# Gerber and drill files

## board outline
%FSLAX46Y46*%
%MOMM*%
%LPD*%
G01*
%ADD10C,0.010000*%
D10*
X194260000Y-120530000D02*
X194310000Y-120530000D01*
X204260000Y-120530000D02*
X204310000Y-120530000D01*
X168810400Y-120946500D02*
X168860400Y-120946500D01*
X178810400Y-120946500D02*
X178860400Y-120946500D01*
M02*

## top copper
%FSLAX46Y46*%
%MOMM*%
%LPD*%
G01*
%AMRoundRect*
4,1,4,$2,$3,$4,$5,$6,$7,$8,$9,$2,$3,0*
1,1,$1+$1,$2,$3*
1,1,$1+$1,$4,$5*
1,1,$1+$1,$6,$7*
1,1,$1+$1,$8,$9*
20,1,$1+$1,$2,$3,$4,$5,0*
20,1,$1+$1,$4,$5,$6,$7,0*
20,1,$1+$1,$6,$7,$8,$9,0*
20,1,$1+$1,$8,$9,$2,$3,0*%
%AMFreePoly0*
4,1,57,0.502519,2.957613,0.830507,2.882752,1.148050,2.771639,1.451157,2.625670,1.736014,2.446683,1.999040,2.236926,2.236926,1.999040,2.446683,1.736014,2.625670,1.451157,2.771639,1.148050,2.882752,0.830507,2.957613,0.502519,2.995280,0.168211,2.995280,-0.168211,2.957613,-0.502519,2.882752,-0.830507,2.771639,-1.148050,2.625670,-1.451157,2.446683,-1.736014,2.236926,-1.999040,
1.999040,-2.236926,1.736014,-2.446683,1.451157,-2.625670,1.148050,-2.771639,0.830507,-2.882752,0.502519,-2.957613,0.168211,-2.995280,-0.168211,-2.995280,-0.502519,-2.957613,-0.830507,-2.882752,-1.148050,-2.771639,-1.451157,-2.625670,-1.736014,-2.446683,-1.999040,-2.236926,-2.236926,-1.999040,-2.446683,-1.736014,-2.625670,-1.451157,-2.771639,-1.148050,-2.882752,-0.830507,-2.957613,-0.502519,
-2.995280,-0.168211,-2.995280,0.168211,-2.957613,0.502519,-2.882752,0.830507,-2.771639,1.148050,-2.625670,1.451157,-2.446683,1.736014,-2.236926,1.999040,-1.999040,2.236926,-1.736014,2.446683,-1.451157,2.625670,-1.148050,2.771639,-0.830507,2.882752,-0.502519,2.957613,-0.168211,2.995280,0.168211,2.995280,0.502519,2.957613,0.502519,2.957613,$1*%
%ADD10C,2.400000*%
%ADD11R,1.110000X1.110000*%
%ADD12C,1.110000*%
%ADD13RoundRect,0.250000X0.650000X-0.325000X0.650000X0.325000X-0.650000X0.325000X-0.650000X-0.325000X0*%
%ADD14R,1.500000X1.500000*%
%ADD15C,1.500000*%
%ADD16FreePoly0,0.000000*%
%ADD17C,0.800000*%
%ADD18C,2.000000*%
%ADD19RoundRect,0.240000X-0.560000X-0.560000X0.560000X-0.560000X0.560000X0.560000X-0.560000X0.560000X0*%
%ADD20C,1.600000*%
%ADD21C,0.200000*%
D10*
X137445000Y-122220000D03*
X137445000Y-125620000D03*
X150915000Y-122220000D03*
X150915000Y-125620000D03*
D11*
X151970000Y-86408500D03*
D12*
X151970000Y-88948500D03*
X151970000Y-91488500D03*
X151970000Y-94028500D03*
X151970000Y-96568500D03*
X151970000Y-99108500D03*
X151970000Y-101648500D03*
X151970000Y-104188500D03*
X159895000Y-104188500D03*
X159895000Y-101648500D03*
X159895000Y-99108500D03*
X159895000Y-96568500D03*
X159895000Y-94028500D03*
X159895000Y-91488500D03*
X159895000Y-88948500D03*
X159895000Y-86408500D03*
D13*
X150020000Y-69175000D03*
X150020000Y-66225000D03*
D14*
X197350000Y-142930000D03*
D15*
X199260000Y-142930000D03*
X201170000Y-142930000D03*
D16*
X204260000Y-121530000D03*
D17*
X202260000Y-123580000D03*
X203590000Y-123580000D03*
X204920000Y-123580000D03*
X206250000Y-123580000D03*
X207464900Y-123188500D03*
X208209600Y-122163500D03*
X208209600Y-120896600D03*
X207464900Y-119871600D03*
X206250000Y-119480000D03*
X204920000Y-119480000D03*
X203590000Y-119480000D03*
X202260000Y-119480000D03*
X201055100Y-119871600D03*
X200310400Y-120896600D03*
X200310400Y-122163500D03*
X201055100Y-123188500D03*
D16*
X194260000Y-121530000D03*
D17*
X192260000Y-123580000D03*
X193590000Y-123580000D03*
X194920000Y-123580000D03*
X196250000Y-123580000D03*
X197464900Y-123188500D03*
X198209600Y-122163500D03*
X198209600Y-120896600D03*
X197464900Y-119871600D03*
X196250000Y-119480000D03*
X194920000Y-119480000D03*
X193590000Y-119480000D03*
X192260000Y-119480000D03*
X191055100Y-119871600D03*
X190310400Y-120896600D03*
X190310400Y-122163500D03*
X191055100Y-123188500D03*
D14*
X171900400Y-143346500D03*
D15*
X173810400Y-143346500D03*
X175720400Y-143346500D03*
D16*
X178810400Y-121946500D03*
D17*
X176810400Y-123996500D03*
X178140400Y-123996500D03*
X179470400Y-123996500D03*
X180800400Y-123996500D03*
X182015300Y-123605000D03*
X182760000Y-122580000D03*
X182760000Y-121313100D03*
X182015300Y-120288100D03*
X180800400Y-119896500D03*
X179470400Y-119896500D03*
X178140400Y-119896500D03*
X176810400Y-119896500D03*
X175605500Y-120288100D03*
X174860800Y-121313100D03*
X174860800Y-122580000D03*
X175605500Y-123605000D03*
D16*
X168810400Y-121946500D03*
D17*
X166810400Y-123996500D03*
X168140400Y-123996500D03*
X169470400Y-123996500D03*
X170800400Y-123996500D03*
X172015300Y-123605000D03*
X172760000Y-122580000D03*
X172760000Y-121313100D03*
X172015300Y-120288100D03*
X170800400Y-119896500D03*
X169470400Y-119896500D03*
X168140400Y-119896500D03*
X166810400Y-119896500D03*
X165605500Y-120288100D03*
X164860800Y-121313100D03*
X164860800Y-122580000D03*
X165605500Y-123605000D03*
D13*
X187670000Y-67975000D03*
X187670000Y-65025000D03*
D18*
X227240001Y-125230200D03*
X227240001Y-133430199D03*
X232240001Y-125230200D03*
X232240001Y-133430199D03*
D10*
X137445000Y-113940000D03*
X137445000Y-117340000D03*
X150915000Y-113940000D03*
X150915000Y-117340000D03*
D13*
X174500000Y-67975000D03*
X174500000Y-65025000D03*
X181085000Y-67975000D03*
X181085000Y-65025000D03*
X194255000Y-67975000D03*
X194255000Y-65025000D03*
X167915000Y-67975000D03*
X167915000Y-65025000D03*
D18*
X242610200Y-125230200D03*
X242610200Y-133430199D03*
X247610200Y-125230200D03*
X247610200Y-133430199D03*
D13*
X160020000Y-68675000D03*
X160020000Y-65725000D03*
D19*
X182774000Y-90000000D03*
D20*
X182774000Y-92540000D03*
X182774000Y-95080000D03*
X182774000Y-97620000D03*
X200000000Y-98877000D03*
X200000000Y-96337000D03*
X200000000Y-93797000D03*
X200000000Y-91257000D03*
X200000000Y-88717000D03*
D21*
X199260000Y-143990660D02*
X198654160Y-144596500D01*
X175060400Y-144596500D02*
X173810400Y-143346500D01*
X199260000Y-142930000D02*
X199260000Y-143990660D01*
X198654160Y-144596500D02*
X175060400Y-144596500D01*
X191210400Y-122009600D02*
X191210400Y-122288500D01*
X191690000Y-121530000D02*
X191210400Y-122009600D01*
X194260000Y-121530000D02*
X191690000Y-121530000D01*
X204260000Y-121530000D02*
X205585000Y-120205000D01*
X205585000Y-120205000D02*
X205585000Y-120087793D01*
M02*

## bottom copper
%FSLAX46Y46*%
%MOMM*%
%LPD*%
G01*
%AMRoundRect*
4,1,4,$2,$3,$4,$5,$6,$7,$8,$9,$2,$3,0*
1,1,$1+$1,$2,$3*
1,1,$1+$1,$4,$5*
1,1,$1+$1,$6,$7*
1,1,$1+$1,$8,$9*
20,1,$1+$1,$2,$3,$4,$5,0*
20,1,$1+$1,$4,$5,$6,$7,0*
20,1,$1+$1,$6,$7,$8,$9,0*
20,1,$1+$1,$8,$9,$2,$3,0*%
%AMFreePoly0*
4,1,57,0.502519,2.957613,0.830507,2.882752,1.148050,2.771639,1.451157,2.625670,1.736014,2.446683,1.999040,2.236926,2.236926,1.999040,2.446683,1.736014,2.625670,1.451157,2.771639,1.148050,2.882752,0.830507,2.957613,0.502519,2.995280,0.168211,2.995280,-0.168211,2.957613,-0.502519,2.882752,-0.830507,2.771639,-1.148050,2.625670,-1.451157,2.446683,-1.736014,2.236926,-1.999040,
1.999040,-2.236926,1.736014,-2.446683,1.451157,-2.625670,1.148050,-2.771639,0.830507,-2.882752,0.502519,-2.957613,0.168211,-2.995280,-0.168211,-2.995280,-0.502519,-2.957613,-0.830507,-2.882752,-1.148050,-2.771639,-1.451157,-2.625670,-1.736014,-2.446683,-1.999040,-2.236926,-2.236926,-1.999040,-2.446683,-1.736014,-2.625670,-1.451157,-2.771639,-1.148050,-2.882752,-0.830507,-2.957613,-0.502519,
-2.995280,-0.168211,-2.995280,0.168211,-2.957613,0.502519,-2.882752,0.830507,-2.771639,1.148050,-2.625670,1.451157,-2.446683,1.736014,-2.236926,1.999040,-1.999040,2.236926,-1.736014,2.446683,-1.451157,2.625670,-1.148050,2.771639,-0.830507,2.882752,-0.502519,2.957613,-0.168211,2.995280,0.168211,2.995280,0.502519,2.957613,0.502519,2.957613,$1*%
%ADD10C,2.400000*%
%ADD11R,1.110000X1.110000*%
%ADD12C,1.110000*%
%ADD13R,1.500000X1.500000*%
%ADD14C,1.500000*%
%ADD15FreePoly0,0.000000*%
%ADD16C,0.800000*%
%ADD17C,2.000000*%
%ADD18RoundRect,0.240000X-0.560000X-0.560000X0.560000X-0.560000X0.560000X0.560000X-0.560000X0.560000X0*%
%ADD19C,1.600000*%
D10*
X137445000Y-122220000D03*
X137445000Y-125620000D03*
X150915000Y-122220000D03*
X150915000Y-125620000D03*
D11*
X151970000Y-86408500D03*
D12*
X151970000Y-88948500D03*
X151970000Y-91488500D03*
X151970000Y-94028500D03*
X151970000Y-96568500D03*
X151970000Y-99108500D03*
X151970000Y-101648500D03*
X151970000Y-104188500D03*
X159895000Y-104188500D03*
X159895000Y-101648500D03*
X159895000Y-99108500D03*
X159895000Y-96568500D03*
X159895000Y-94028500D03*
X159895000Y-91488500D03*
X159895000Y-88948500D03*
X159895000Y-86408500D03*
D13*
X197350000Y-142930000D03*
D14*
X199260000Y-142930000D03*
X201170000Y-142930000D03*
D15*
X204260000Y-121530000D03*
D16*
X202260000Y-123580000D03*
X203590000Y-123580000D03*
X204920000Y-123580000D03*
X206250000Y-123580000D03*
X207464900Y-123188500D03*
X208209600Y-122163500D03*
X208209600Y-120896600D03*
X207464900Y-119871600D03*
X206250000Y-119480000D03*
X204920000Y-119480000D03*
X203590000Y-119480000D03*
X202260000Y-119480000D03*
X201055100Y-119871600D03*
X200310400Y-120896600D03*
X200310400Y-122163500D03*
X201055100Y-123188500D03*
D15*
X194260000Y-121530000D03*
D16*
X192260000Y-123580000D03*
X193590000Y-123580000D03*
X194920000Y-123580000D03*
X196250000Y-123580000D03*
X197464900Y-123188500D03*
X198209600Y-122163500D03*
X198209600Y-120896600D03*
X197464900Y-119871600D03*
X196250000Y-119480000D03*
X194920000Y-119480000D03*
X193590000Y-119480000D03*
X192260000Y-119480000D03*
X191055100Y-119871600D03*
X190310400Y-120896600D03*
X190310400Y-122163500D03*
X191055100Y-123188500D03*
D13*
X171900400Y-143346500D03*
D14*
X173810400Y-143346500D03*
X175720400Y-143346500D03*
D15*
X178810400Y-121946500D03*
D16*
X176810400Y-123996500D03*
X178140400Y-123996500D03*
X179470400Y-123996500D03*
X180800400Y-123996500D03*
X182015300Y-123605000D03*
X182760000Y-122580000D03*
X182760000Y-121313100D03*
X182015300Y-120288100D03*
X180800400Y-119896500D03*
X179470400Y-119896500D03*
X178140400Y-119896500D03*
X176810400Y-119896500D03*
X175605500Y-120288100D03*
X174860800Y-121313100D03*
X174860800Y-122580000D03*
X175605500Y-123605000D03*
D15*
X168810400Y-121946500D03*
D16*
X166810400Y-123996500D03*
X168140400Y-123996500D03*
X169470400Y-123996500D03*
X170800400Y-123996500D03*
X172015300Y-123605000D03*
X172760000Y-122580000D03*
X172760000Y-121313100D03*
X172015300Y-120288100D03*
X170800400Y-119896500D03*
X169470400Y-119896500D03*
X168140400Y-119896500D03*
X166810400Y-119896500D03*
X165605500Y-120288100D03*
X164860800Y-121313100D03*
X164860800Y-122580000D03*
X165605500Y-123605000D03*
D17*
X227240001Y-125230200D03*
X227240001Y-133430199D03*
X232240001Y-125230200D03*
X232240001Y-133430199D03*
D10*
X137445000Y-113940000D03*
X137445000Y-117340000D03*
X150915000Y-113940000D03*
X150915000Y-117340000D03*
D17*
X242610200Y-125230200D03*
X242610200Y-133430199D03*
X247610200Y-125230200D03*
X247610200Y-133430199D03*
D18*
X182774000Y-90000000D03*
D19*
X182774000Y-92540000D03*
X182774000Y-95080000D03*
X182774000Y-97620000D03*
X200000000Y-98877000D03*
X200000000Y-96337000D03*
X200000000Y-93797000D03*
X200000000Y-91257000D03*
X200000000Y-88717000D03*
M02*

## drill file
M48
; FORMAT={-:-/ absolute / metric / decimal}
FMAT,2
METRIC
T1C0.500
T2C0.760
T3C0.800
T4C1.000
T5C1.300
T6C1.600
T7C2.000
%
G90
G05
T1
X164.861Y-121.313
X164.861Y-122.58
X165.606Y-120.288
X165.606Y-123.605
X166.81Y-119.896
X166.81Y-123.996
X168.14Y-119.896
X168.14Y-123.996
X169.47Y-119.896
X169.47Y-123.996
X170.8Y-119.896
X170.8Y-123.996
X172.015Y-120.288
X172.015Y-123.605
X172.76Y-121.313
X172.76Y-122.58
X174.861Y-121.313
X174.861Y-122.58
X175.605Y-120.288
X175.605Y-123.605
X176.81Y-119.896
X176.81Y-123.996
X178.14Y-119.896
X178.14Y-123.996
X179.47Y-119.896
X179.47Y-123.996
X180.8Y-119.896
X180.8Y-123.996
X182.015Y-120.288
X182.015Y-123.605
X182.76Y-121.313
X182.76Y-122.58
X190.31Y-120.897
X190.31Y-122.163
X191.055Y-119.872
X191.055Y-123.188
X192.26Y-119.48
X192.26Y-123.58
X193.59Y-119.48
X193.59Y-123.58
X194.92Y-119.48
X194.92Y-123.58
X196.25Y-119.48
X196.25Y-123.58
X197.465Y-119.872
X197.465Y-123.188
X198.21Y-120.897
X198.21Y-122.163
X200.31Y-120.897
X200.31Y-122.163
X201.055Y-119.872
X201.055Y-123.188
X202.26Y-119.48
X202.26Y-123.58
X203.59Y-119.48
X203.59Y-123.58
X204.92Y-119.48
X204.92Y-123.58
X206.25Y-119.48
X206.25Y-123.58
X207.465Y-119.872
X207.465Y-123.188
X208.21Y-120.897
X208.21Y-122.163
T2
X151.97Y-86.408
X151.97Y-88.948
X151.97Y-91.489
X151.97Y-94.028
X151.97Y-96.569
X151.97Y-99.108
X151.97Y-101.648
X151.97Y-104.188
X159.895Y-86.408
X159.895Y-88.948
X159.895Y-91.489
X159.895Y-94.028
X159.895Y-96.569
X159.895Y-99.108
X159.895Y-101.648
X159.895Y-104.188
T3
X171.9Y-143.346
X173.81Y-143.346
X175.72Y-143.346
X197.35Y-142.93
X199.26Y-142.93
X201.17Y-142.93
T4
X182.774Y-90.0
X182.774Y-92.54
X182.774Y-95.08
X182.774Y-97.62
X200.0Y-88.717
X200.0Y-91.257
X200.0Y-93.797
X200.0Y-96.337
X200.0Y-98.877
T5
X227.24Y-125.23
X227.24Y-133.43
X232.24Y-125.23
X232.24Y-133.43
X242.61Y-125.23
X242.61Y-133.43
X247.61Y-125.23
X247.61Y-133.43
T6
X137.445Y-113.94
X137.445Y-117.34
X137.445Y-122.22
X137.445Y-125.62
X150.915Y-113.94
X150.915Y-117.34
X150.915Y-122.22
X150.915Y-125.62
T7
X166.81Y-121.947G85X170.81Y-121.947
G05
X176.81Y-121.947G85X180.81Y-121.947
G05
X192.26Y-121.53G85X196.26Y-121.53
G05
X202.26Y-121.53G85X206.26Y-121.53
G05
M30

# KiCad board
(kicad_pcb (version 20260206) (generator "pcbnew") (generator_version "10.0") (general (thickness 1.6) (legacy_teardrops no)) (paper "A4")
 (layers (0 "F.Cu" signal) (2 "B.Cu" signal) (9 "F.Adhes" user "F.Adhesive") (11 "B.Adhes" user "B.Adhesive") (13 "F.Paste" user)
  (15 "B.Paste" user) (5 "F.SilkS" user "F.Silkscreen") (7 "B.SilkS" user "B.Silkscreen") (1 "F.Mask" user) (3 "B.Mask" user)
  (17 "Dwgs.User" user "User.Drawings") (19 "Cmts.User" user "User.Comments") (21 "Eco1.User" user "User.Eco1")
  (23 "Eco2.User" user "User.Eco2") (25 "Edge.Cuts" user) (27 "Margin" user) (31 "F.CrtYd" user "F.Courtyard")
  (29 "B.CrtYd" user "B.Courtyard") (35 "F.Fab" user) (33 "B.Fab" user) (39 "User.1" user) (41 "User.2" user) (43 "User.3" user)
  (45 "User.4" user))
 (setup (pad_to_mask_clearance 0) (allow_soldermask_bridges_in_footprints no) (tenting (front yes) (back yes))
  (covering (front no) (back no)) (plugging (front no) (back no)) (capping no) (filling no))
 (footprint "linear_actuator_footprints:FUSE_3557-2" (layer "F.Cu") (at 144.18 123.92)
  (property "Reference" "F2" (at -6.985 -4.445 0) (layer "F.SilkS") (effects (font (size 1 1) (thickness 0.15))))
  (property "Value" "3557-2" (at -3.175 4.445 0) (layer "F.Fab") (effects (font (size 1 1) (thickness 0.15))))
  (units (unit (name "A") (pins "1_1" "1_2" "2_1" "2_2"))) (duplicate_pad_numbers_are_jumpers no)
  (pad "1_1" thru_hole circle (at -6.735 -1.7) (size 2.4 2.4) (drill 1.6) (layers "*.Cu" "*.Mask") (remove_unused_layers no)
   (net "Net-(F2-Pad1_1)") (solder_mask_margin 0.102))
  (pad "1_2" thru_hole circle (at -6.735 1.7) (size 2.4 2.4) (drill 1.6) (layers "*.Cu" "*.Mask") (remove_unused_layers no)
   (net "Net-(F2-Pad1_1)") (solder_mask_margin 0.102))
  (pad "2_1" thru_hole circle (at 6.735 -1.7) (size 2.4 2.4) (drill 1.6) (layers "*.Cu" "*.Mask") (remove_unused_layers no)
   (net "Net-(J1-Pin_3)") (solder_mask_margin 0.102))
  (pad "2_2" thru_hole circle (at 6.735 1.7) (size 2.4 2.4) (drill 1.6) (layers "*.Cu" "*.Mask") (remove_unused_layers no)
   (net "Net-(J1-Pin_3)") (solder_mask_margin 0.102)))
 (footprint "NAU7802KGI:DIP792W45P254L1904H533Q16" (layer "F.Cu") (at 155.9325 95.2985)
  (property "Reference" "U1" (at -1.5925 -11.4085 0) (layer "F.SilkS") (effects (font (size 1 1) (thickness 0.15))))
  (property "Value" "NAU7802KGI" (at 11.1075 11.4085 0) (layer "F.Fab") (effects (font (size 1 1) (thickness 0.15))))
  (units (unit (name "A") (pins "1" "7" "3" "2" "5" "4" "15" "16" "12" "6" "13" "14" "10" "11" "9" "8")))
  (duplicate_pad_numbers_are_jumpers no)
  (pad "1" thru_hole rect (at -3.9625 -8.89) (size 1.11 1.11) (drill 0.76) (layers "*.Cu" "*.Mask") (remove_unused_layers no) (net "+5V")
   (solder_mask_margin 0.102))
  (pad "2" thru_hole circle (at -3.9625 -6.35) (size 1.11 1.11) (drill 0.76) (layers "*.Cu" "*.Mask") (remove_unused_layers no) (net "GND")
   (solder_mask_margin 0.102))
  (pad "3" thru_hole circle (at -3.9625 -3.81) (size 1.11 1.11) (drill 0.76) (layers "*.Cu" "*.Mask") (remove_unused_layers no)
   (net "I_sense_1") (solder_mask_margin 0.102))
  (pad "4" thru_hole circle (at -3.9625 -1.27) (size 1.11 1.11) (drill 0.76) (layers "*.Cu" "*.Mask") (remove_unused_layers no) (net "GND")
   (solder_mask_margin 0.102))
  (pad "5" thru_hole circle (at -3.9625 1.27) (size 1.11 1.11) (drill 0.76) (layers "*.Cu" "*.Mask") (remove_unused_layers no)
   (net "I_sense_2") (solder_mask_margin 0.102))
  (pad "6" thru_hole circle (at -3.9625 3.81) (size 1.11 1.11) (drill 0.76) (layers "*.Cu" "*.Mask") (remove_unused_layers no)
   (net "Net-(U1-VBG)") (solder_mask_margin 0.102))
  (pad "7" thru_hole circle (at -3.9625 6.35) (size 1.11 1.11) (drill 0.76) (layers "*.Cu" "*.Mask") (remove_unused_layers no) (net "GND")
   (solder_mask_margin 0.102))
  (pad "8" thru_hole circle (at -3.9625 8.89) (size 1.11 1.11) (drill 0.76) (layers "*.Cu" "*.Mask") (remove_unused_layers no) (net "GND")
   (solder_mask_margin 0.102))
  (pad "9" thru_hole circle (at 3.9625 8.89) (size 1.11 1.11) (drill 0.76) (layers "*.Cu" "*.Mask") (remove_unused_layers no) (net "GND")
   (solder_mask_margin 0.102))
  (pad "10" thru_hole circle (at 3.9625 6.35) (size 1.11 1.11) (drill 0.76) (layers "*.Cu" "*.Mask") (remove_unused_layers no)
   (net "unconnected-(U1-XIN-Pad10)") (solder_mask_margin 0.102))
  (pad "11" thru_hole circle (at 3.9625 3.81) (size 1.11 1.11) (drill 0.76) (layers "*.Cu" "*.Mask") (remove_unused_layers no)
   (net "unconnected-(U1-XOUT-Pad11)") (solder_mask_margin 0.102))
  (pad "12" thru_hole circle (at 3.9625 1.27) (size 1.11 1.11) (drill 0.76) (layers "*.Cu" "*.Mask") (remove_unused_layers no)
   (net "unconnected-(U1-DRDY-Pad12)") (solder_mask_margin 0.102))
  (pad "13" thru_hole circle (at 3.9625 -1.27) (size 1.11 1.11) (drill 0.76) (layers "*.Cu" "*.Mask") (remove_unused_layers no)
   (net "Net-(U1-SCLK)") (solder_mask_margin 0.102))
  (pad "14" thru_hole circle (at 3.9625 -3.81) (size 1.11 1.11) (drill 0.76) (layers "*.Cu" "*.Mask") (remove_unused_layers no)
   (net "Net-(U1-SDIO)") (solder_mask_margin 0.102))
  (pad "15" thru_hole circle (at 3.9625 -6.35) (size 1.11 1.11) (drill 0.76) (layers "*.Cu" "*.Mask") (remove_unused_layers no) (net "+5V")
   (solder_mask_margin 0.102))
  (pad "16" thru_hole circle (at 3.9625 -8.89) (size 1.11 1.11) (drill 0.76) (layers "*.Cu" "*.Mask") (remove_unused_layers no)
   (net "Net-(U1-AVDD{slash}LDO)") (solder_mask_margin 0.102)))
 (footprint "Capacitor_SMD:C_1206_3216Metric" (layer "F.Cu") (at 150.02 67.7 90)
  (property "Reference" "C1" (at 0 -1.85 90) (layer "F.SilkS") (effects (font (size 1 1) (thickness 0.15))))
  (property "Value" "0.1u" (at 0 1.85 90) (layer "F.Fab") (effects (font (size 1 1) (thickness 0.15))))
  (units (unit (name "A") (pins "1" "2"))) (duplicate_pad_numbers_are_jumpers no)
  (pad "1" smd roundrect (at -1.475 0 90) (size 1.15 1.8) (layers "F.Cu" "F.Mask" "F.Paste") (roundrect_rratio 0.217391) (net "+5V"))
  (pad "2" smd roundrect (at 1.475 0 90) (size 1.15 1.8) (layers "F.Cu" "F.Mask" "F.Paste") (roundrect_rratio 0.217391) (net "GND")))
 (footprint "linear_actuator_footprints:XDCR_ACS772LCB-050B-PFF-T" (layer "F.Cu") (at 199.26 132.23)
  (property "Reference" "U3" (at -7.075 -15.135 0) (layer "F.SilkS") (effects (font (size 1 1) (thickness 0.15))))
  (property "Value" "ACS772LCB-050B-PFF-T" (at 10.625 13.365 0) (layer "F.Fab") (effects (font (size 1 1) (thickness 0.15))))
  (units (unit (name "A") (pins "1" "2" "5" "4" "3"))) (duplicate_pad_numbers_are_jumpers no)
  (fp_line (start -5 -11.7) (end -4.95 -11.7) (stroke (width 0.01) (type solid)) (layer "Edge.Cuts"))
  (fp_line (start 5 -11.7) (end 5.05 -11.7) (stroke (width 0.01) (type solid)) (layer "Edge.Cuts"))
  (pad "1" thru_hole rect (at -1.91 10.7) (size 1.5 1.5) (drill 0.8) (layers "*.Cu" "*.Mask") (remove_unused_layers no) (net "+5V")
   (solder_mask_margin 0.102))
  (pad "2" thru_hole circle (at 0 10.7) (size 1.5 1.5) (drill 0.8) (layers "*.Cu" "*.Mask") (remove_unused_layers no) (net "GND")
   (solder_mask_margin 0.102))
  (pad "3" thru_hole circle (at 1.91 10.7) (size 1.5 1.5) (drill 0.8) (layers "*.Cu" "*.Mask") (remove_unused_layers no) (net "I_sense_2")
   (solder_mask_margin 0.102))
  (pad "4" thru_hole custom (at 5 -10.7) (size 6 3) (drill oval 6 2) (layers "*.Cu") (remove_unused_layers no) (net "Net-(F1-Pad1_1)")
   (thermal_bridge_angle 90) (options (clearance outline) (anchor circle)) (primitives))
  (pad "4_1" thru_hole circle (at 3 -8.65) (size 0.8 0.8) (drill 0.5) (layers "*.Cu" "*.Mask") (remove_unused_layers no)
   (solder_mask_margin 0.102))
  (pad "4_2" thru_hole circle (at 4.33 -8.65) (size 0.8 0.8) (drill 0.5) (layers "*.Cu" "*.Mask") (remove_unused_layers no)
   (solder_mask_margin 0.102))
  (pad "4_3" thru_hole circle (at 5.66 -8.65) (size 0.8 0.8) (drill 0.5) (layers "*.Cu" "*.Mask") (remove_unused_layers no)
   (solder_mask_margin 0.102))
  (pad "4_4" thru_hole circle (at 6.99 -8.65) (size 0.8 0.8) (drill 0.5) (layers "*.Cu" "*.Mask") (remove_unused_layers no)
   (solder_mask_margin 0.102))
  (pad "4_5" thru_hole circle (at 8.2049 -9.0415) (size 0.8 0.8) (drill 0.5) (layers "*.Cu" "*.Mask") (remove_unused_layers no)
   (solder_mask_margin 0.102))
  (pad "4_6" thru_hole circle (at 8.9496 -10.0665) (size 0.8 0.8) (drill 0.5) (layers "*.Cu" "*.Mask") (remove_unused_layers no)
   (solder_mask_margin 0.102))
  (pad "4_7" thru_hole circle (at 8.9496 -11.3334) (size 0.8 0.8) (drill 0.5) (layers "*.Cu" "*.Mask") (remove_unused_layers no)
   (solder_mask_margin 0.102))
  (pad "4_8" thru_hole circle (at 8.2049 -12.3584) (size 0.8 0.8) (drill 0.5) (layers "*.Cu" "*.Mask") (remove_unused_layers no)
   (solder_mask_margin 0.102))
  (pad "4_9" thru_hole circle (at 6.99 -12.75) (size 0.8 0.8) (drill 0.5) (layers "*.Cu" "*.Mask") (remove_unused_layers no)
   (solder_mask_margin 0.102))
  (pad "4_10" thru_hole circle (at 5.66 -12.75) (size 0.8 0.8) (drill 0.5) (layers "*.Cu" "*.Mask") (remove_unused_layers no)
   (solder_mask_margin 0.102))
  (pad "4_11" thru_hole circle (at 4.33 -12.75) (size 0.8 0.8) (drill 0.5) (layers "*.Cu" "*.Mask") (remove_unused_layers no)
   (solder_mask_margin 0.102))
  (pad "4_12" thru_hole circle (at 3 -12.75) (size 0.8 0.8) (drill 0.5) (layers "*.Cu" "*.Mask") (remove_unused_layers no)
   (solder_mask_margin 0.102))
  (pad "4_13" thru_hole circle (at 1.7951 -12.3584) (size 0.8 0.8) (drill 0.5) (layers "*.Cu" "*.Mask") (remove_unused_layers no)
   (solder_mask_margin 0.102))
  (pad "4_14" thru_hole circle (at 1.0504 -11.3334) (size 0.8 0.8) (drill 0.5) (layers "*.Cu" "*.Mask") (remove_unused_layers no)
   (solder_mask_margin 0.102))
  (pad "4_15" thru_hole circle (at 1.0504 -10.0665) (size 0.8 0.8) (drill 0.5) (layers "*.Cu" "*.Mask") (remove_unused_layers no)
   (solder_mask_margin 0.102))
  (pad "4_16" thru_hole circle (at 1.7951 -9.0415) (size 0.8 0.8) (drill 0.5) (layers "*.Cu" "*.Mask") (remove_unused_layers no)
   (solder_mask_margin 0.102))
  (pad "5" thru_hole custom (at -5 -10.7) (size 6 3) (drill oval 6 2) (layers "*.Cu") (remove_unused_layers no) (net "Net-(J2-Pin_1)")
   (thermal_bridge_angle 90) (options (clearance outline) (anchor circle)) (primitives))
  (pad "5_1" thru_hole circle (at -7 -8.65) (size 0.8 0.8) (drill 0.5) (layers "*.Cu" "*.Mask") (remove_unused_layers no)
   (solder_mask_margin 0.102))
  (pad "5_2" thru_hole circle (at -5.67 -8.65) (size 0.8 0.8) (drill 0.5) (layers "*.Cu" "*.Mask") (remove_unused_layers no)
   (solder_mask_margin 0.102))
  (pad "5_3" thru_hole circle (at -4.34 -8.65) (size 0.8 0.8) (drill 0.5) (layers "*.Cu" "*.Mask") (remove_unused_layers no)
   (solder_mask_margin 0.102))
  (pad "5_4" thru_hole circle (at -3.01 -8.65) (size 0.8 0.8) (drill 0.5) (layers "*.Cu" "*.Mask") (remove_unused_layers no)
   (solder_mask_margin 0.102))
  (pad "5_5" thru_hole circle (at -1.7951 -9.0415) (size 0.8 0.8) (drill 0.5) (layers "*.Cu" "*.Mask") (remove_unused_layers no)
   (solder_mask_margin 0.102))
  (pad "5_6" thru_hole circle (at -1.0504 -10.0665) (size 0.8 0.8) (drill 0.5) (layers "*.Cu" "*.Mask") (remove_unused_layers no)
   (solder_mask_margin 0.102))
  (pad "5_7" thru_hole circle (at -1.0504 -11.3334) (size 0.8 0.8) (drill 0.5) (layers "*.Cu" "*.Mask") (remove_unused_layers no)
   (solder_mask_margin 0.102))
  (pad "5_8" thru_hole circle (at -1.7951 -12.3584) (size 0.8 0.8) (drill 0.5) (layers "*.Cu" "*.Mask") (remove_unused_layers no)
   (solder_mask_margin 0.102))
  (pad "5_9" thru_hole circle (at -3.01 -12.75) (size 0.8 0.8) (drill 0.5) (layers "*.Cu" "*.Mask") (remove_unused_layers no)
   (solder_mask_margin 0.102))
  (pad "5_10" thru_hole circle (at -4.34 -12.75) (size 0.8 0.8) (drill 0.5) (layers "*.Cu" "*.Mask") (remove_unused_layers no)
   (solder_mask_margin 0.102))
  (pad "5_11" thru_hole circle (at -5.67 -12.75) (size 0.8 0.8) (drill 0.5) (layers "*.Cu" "*.Mask") (remove_unused_layers no)
   (solder_mask_margin 0.102))
  (pad "5_12" thru_hole circle (at -7 -12.75) (size 0.8 0.8) (drill 0.5) (layers "*.Cu" "*.Mask") (remove_unused_layers no)
   (solder_mask_margin 0.102))
  (pad "5_13" thru_hole circle (at -8.2049 -12.3584) (size 0.8 0.8) (drill 0.5) (layers "*.Cu" "*.Mask") (remove_unused_layers no)
   (solder_mask_margin 0.102))
  (pad "5_14" thru_hole circle (at -8.9496 -11.3334) (size 0.8 0.8) (drill 0.5) (layers "*.Cu" "*.Mask") (remove_unused_layers no)
   (solder_mask_margin 0.102))
  (pad "5_15" thru_hole circle (at -8.9496 -10.0665) (size 0.8 0.8) (drill 0.5) (layers "*.Cu" "*.Mask") (remove_unused_layers no)
   (solder_mask_margin 0.102))
  (pad "5_16" thru_hole circle (at -8.2049 -9.0415) (size 0.8 0.8) (drill 0.5) (layers "*.Cu" "*.Mask") (remove_unused_layers no)
   (solder_mask_margin 0.102)))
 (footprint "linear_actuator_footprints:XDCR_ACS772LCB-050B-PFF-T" (layer "F.Cu") (at 173.8104 132.6465)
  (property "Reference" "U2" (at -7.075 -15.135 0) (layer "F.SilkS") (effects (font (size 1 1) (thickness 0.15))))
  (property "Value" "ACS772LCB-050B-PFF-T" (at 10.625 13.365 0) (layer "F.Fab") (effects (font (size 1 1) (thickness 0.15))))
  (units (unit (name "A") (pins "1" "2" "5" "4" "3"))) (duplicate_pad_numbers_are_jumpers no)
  (fp_line (start -5 -11.7) (end -4.95 -11.7) (stroke (width 0.01) (type solid)) (layer "Edge.Cuts"))
  (fp_line (start 5 -11.7) (end 5.05 -11.7) (stroke (width 0.01) (type solid)) (layer "Edge.Cuts"))
  (pad "1" thru_hole rect (at -1.91 10.7) (size 1.5 1.5) (drill 0.8) (layers "*.Cu" "*.Mask") (remove_unused_layers no) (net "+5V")
   (solder_mask_margin 0.102))
  (pad "2" thru_hole circle (at 0 10.7) (size 1.5 1.5) (drill 0.8) (layers "*.Cu" "*.Mask") (remove_unused_layers no) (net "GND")
   (solder_mask_margin 0.102))
  (pad "3" thru_hole circle (at 1.91 10.7) (size 1.5 1.5) (drill 0.8) (layers "*.Cu" "*.Mask") (remove_unused_layers no) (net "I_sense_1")
   (solder_mask_margin 0.102))
  (pad "4" thru_hole custom (at 5 -10.7) (size 6 3) (drill oval 6 2) (layers "*.Cu") (remove_unused_layers no) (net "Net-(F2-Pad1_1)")
   (thermal_bridge_angle 90) (options (clearance outline) (anchor circle)) (primitives))
  (pad "4_1" thru_hole circle (at 3 -8.65) (size 0.8 0.8) (drill 0.5) (layers "*.Cu" "*.Mask") (remove_unused_layers no)
   (solder_mask_margin 0.102))
  (pad "4_2" thru_hole circle (at 4.33 -8.65) (size 0.8 0.8) (drill 0.5) (layers "*.Cu" "*.Mask") (remove_unused_layers no)
   (solder_mask_margin 0.102))
  (pad "4_3" thru_hole circle (at 5.66 -8.65) (size 0.8 0.8) (drill 0.5) (layers "*.Cu" "*.Mask") (remove_unused_layers no)
   (solder_mask_margin 0.102))
  (pad "4_4" thru_hole circle (at 6.99 -8.65) (size 0.8 0.8) (drill 0.5) (layers "*.Cu" "*.Mask") (remove_unused_layers no)
   (solder_mask_margin 0.102))
  (pad "4_5" thru_hole circle (at 8.2049 -9.0415) (size 0.8 0.8) (drill 0.5) (layers "*.Cu" "*.Mask") (remove_unused_layers no)
   (solder_mask_margin 0.102))
  (pad "4_6" thru_hole circle (at 8.9496 -10.0665) (size 0.8 0.8) (drill 0.5) (layers "*.Cu" "*.Mask") (remove_unused_layers no)
   (solder_mask_margin 0.102))
  (pad "4_7" thru_hole circle (at 8.9496 -11.3334) (size 0.8 0.8) (drill 0.5) (layers "*.Cu" "*.Mask") (remove_unused_layers no)
   (solder_mask_margin 0.102))
  (pad "4_8" thru_hole circle (at 8.2049 -12.3584) (size 0.8 0.8) (drill 0.5) (layers "*.Cu" "*.Mask") (remove_unused_layers no)
   (solder_mask_margin 0.102))
  (pad "4_9" thru_hole circle (at 6.99 -12.75) (size 0.8 0.8) (drill 0.5) (layers "*.Cu" "*.Mask") (remove_unused_layers no)
   (solder_mask_margin 0.102))
  (pad "4_10" thru_hole circle (at 5.66 -12.75) (size 0.8 0.8) (drill 0.5) (layers "*.Cu" "*.Mask") (remove_unused_layers no)
   (solder_mask_margin 0.102))
  (pad "4_11" thru_hole circle (at 4.33 -12.75) (size 0.8 0.8) (drill 0.5) (layers "*.Cu" "*.Mask") (remove_unused_layers no)
   (solder_mask_margin 0.102))
  (pad "4_12" thru_hole circle (at 3 -12.75) (size 0.8 0.8) (drill 0.5) (layers "*.Cu" "*.Mask") (remove_unused_layers no)
   (solder_mask_margin 0.102))
  (pad "4_13" thru_hole circle (at 1.7951 -12.3584) (size 0.8 0.8) (drill 0.5) (layers "*.Cu" "*.Mask") (remove_unused_layers no)
   (solder_mask_margin 0.102))
  (pad "4_14" thru_hole circle (at 1.0504 -11.3334) (size 0.8 0.8) (drill 0.5) (layers "*.Cu" "*.Mask") (remove_unused_layers no)
   (solder_mask_margin 0.102))
  (pad "4_15" thru_hole circle (at 1.0504 -10.0665) (size 0.8 0.8) (drill 0.5) (layers "*.Cu" "*.Mask") (remove_unused_layers no)
   (solder_mask_margin 0.102))
  (pad "4_16" thru_hole circle (at 1.7951 -9.0415) (size 0.8 0.8) (drill 0.5) (layers "*.Cu" "*.Mask") (remove_unused_layers no)
   (solder_mask_margin 0.102))
  (pad "5" thru_hole custom (at -5 -10.7) (size 6 3) (drill oval 6 2) (layers "*.Cu") (remove_unused_layers no) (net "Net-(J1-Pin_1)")
   (thermal_bridge_angle 90) (options (clearance outline) (anchor circle)) (primitives))
  (pad "5_1" thru_hole circle (at -7 -8.65) (size 0.8 0.8) (drill 0.5) (layers "*.Cu" "*.Mask") (remove_unused_layers no)
   (solder_mask_margin 0.102))
  (pad "5_2" thru_hole circle (at -5.67 -8.65) (size 0.8 0.8) (drill 0.5) (layers "*.Cu" "*.Mask") (remove_unused_layers no)
   (solder_mask_margin 0.102))
  (pad "5_3" thru_hole circle (at -4.34 -8.65) (size 0.8 0.8) (drill 0.5) (layers "*.Cu" "*.Mask") (remove_unused_layers no)
   (solder_mask_margin 0.102))
  (pad "5_4" thru_hole circle (at -3.01 -8.65) (size 0.8 0.8) (drill 0.5) (layers "*.Cu" "*.Mask") (remove_unused_layers no)
   (solder_mask_margin 0.102))
  (pad "5_5" thru_hole circle (at -1.7951 -9.0415) (size 0.8 0.8) (drill 0.5) (layers "*.Cu" "*.Mask") (remove_unused_layers no)
   (solder_mask_margin 0.102))
  (pad "5_6" thru_hole circle (at -1.0504 -10.0665) (size 0.8 0.8) (drill 0.5) (layers "*.Cu" "*.Mask") (remove_unused_layers no)
   (solder_mask_margin 0.102))
  (pad "5_7" thru_hole circle (at -1.0504 -11.3334) (size 0.8 0.8) (drill 0.5) (layers "*.Cu" "*.Mask") (remove_unused_layers no)
   (solder_mask_margin 0.102))
  (pad "5_8" thru_hole circle (at -1.7951 -12.3584) (size 0.8 0.8) (drill 0.5) (layers "*.Cu" "*.Mask") (remove_unused_layers no)
   (solder_mask_margin 0.102))
  (pad "5_9" thru_hole circle (at -3.01 -12.75) (size 0.8 0.8) (drill 0.5) (layers "*.Cu" "*.Mask") (remove_unused_layers no)
   (solder_mask_margin 0.102))
  (pad "5_10" thru_hole circle (at -4.34 -12.75) (size 0.8 0.8) (drill 0.5) (layers "*.Cu" "*.Mask") (remove_unused_layers no)
   (solder_mask_margin 0.102))
  (pad "5_11" thru_hole circle (at -5.67 -12.75) (size 0.8 0.8) (drill 0.5) (layers "*.Cu" "*.Mask") (remove_unused_layers no)
   (solder_mask_margin 0.102))
  (pad "5_12" thru_hole circle (at -7 -12.75) (size 0.8 0.8) (drill 0.5) (layers "*.Cu" "*.Mask") (remove_unused_layers no)
   (solder_mask_margin 0.102))
  (pad "5_13" thru_hole circle (at -8.2049 -12.3584) (size 0.8 0.8) (drill 0.5) (layers "*.Cu" "*.Mask") (remove_unused_layers no)
   (solder_mask_margin 0.102))
  (pad "5_14" thru_hole circle (at -8.9496 -11.3334) (size 0.8 0.8) (drill 0.5) (layers "*.Cu" "*.Mask") (remove_unused_layers no)
   (solder_mask_margin 0.102))
  (pad "5_15" thru_hole circle (at -8.9496 -10.0665) (size 0.8 0.8) (drill 0.5) (layers "*.Cu" "*.Mask") (remove_unused_layers no)
   (solder_mask_margin 0.102))
  (pad "5_16" thru_hole circle (at -8.2049 -9.0415) (size 0.8 0.8) (drill 0.5) (layers "*.Cu" "*.Mask") (remove_unused_layers no)
   (solder_mask_margin 0.102)))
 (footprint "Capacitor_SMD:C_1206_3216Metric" (layer "F.Cu") (at 187.67 66.5 90)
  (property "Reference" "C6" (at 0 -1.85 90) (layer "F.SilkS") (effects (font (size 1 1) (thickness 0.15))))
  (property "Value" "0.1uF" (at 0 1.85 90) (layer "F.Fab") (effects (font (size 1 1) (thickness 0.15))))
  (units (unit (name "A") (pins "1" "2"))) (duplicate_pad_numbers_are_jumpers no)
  (pad "1" smd roundrect (at -1.475 0 90) (size 1.15 1.8) (layers "F.Cu" "F.Mask" "F.Paste") (roundrect_rratio 0.217391) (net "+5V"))
  (pad "2" smd roundrect (at 1.475 0 90) (size 1.15 1.8) (layers "F.Cu" "F.Mask" "F.Paste") (roundrect_rratio 0.217391) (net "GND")))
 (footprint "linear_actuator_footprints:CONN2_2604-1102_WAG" (layer "F.Cu") (at 227.240001 125.2302)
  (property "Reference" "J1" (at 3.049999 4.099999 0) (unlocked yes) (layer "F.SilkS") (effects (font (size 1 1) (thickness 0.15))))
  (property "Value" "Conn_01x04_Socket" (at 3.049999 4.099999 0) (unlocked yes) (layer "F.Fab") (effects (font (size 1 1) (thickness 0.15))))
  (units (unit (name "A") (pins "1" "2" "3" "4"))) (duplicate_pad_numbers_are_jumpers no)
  (pad "1" thru_hole circle (at 0 0) (size 2 2) (drill 1.3) (layers "*.Cu" "*.Mask") (remove_unused_layers no) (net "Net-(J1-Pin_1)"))
  (pad "2" thru_hole circle (at 0 8.199999) (size 2 2) (drill 1.3) (layers "*.Cu" "*.Mask") (remove_unused_layers no) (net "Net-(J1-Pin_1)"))
  (pad "3" thru_hole circle (at 5 0) (size 2 2) (drill 1.3) (layers "*.Cu" "*.Mask") (remove_unused_layers no) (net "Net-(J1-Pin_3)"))
  (pad "4" thru_hole circle (at 5 8.199999) (size 2 2) (drill 1.3) (layers "*.Cu" "*.Mask") (remove_unused_layers no) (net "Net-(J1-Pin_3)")))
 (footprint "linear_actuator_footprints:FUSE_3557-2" (layer "F.Cu") (at 144.18 115.64)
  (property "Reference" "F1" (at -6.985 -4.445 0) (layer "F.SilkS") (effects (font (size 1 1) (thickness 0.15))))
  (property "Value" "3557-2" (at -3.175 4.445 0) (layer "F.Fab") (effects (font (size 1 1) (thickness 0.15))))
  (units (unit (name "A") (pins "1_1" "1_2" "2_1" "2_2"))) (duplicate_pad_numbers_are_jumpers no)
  (pad "1_1" thru_hole circle (at -6.735 -1.7) (size 2.4 2.4) (drill 1.6) (layers "*.Cu" "*.Mask") (remove_unused_layers no)
   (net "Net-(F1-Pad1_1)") (solder_mask_margin 0.102))
  (pad "1_2" thru_hole circle (at -6.735 1.7) (size 2.4 2.4) (drill 1.6) (layers "*.Cu" "*.Mask") (remove_unused_layers no)
   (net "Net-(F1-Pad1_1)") (solder_mask_margin 0.102))
  (pad "2_1" thru_hole circle (at 6.735 -1.7) (size 2.4 2.4) (drill 1.6) (layers "*.Cu" "*.Mask") (remove_unused_layers no)
   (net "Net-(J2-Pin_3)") (solder_mask_margin 0.102))
  (pad "2_2" thru_hole circle (at 6.735 1.7) (size 2.4 2.4) (drill 1.6) (layers "*.Cu" "*.Mask") (remove_unused_layers no)
   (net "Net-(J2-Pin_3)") (solder_mask_margin 0.102)))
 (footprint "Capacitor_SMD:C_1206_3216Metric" (layer "F.Cu") (at 174.5 66.5 90)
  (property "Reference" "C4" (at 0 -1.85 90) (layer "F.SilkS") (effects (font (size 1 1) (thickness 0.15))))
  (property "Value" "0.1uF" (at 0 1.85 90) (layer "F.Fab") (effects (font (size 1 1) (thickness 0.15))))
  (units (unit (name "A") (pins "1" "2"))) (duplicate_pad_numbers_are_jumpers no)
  (pad "1" smd roundrect (at -1.475 0 90) (size 1.15 1.8) (layers "F.Cu" "F.Mask" "F.Paste") (roundrect_rratio 0.217391) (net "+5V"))
  (pad "2" smd roundrect (at 1.475 0 90) (size 1.15 1.8) (layers "F.Cu" "F.Mask" "F.Paste") (roundrect_rratio 0.217391) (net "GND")))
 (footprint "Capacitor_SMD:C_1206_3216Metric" (layer "F.Cu") (at 181.085 66.5 90)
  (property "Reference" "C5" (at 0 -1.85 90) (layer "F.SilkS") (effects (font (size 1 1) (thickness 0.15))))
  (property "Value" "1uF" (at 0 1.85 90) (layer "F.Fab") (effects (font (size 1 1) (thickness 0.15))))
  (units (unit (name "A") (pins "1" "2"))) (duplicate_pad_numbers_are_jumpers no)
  (pad "1" smd roundrect (at -1.475 0 90) (size 1.15 1.8) (layers "F.Cu" "F.Mask" "F.Paste") (roundrect_rratio 0.217391) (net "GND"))
  (pad "2" smd roundrect (at 1.475 0 90) (size 1.15 1.8) (layers "F.Cu" "F.Mask" "F.Paste") (roundrect_rratio 0.217391)
   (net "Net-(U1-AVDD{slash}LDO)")))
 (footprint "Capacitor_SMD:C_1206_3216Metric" (layer "F.Cu") (at 194.255 66.5 90)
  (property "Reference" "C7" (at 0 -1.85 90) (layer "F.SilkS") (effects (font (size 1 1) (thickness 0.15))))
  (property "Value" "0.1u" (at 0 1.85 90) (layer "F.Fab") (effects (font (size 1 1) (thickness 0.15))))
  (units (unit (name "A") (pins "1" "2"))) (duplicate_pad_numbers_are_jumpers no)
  (pad "1" smd roundrect (at -1.475 0 90) (size 1.15 1.8) (layers "F.Cu" "F.Mask" "F.Paste") (roundrect_rratio 0.217391)
   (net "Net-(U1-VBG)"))
  (pad "2" smd roundrect (at 1.475 0 90) (size 1.15 1.8) (layers "F.Cu" "F.Mask" "F.Paste") (roundrect_rratio 0.217391) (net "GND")))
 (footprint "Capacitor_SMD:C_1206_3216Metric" (layer "F.Cu") (at 167.915 66.5 90)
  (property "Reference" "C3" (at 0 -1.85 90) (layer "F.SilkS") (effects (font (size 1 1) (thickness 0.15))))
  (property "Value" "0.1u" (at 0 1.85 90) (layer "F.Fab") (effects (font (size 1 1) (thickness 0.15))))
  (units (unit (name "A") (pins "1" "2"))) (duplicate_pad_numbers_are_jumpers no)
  (pad "1" smd roundrect (at -1.475 0 90) (size 1.15 1.8) (layers "F.Cu" "F.Mask" "F.Paste") (roundrect_rratio 0.217391)
   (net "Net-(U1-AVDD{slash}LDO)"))
  (pad "2" smd roundrect (at 1.475 0 90) (size 1.15 1.8) (layers "F.Cu" "F.Mask" "F.Paste") (roundrect_rratio 0.217391) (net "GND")))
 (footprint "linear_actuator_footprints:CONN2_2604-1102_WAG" (layer "F.Cu") (at 242.6102 125.2302)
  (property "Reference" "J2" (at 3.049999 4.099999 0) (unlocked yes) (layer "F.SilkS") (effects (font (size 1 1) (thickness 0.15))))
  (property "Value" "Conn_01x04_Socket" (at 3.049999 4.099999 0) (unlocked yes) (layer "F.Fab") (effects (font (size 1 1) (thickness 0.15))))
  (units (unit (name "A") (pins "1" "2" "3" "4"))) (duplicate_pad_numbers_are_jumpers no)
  (pad "1" thru_hole circle (at 0 0) (size 2 2) (drill 1.3) (layers "*.Cu" "*.Mask") (remove_unused_layers no) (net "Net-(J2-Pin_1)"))
  (pad "2" thru_hole circle (at 0 8.199999) (size 2 2) (drill 1.3) (layers "*.Cu" "*.Mask") (remove_unused_layers no) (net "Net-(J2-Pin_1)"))
  (pad "3" thru_hole circle (at 5 0) (size 2 2) (drill 1.3) (layers "*.Cu" "*.Mask") (remove_unused_layers no) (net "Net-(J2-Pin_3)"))
  (pad "4" thru_hole circle (at 5 8.199999) (size 2 2) (drill 1.3) (layers "*.Cu" "*.Mask") (remove_unused_layers no) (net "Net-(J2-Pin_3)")))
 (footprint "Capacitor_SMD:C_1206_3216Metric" (layer "F.Cu") (at 160.02 67.2 90)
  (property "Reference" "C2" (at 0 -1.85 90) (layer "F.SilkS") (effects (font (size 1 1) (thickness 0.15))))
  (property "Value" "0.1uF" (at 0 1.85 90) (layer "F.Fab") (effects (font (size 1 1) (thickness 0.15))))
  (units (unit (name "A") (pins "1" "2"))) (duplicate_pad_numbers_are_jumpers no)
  (pad "1" smd roundrect (at -1.475 0 90) (size 1.15 1.8) (layers "F.Cu" "F.Mask" "F.Paste") (roundrect_rratio 0.217391) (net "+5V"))
  (pad "2" smd roundrect (at 1.475 0 90) (size 1.15 1.8) (layers "F.Cu" "F.Mask" "F.Paste") (roundrect_rratio 0.217391) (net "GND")))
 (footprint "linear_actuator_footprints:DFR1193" (layer "F.Cu") (at 182.774 90)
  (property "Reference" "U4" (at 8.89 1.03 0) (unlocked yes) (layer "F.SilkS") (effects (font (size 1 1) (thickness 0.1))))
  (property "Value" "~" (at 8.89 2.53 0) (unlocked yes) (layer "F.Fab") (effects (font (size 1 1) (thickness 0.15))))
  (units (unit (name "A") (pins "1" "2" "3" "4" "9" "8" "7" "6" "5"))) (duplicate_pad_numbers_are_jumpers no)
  (pad "1" thru_hole roundrect (at 0 0) (size 1.6 1.6) (drill 1) (layers "*.Cu" "*.Mask") (remove_unused_layers no) (roundrect_rratio 0.15)
   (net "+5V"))
  (pad "2" thru_hole circle (at 0 2.54) (size 1.6 1.6) (drill 1) (layers "*.Cu" "*.Mask") (remove_unused_layers no) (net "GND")
   (thermal_bridge_angle 90))
  (pad "3" thru_hole circle (at 0 5.08) (size 1.6 1.6) (drill 1) (layers "*.Cu" "*.Mask") (remove_unused_layers no) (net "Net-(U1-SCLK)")
   (thermal_bridge_angle 90))
  (pad "4" thru_hole circle (at 0 7.62) (size 1.6 1.6) (drill 1) (layers "*.Cu" "*.Mask") (remove_unused_layers no) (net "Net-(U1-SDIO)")
   (thermal_bridge_angle 90))
  (pad "5" thru_hole circle (at 17.226 8.877) (size 1.6 1.6) (drill 1) (layers "*.Cu" "*.Mask") (remove_unused_layers no)
   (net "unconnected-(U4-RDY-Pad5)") (thermal_bridge_angle 90))
  (pad "6" thru_hole circle (at 17.226 6.337) (size 1.6 1.6) (drill 1) (layers "*.Cu" "*.Mask") (remove_unused_layers no)
   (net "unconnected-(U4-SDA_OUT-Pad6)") (thermal_bridge_angle 90))
  (pad "7" thru_hole circle (at 17.226 3.797) (size 1.6 1.6) (drill 1) (layers "*.Cu" "*.Mask") (remove_unused_layers no)
   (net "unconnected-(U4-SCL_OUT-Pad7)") (thermal_bridge_angle 90))
  (pad "8" thru_hole circle (at 17.226 1.257) (size 1.6 1.6) (drill 1) (layers "*.Cu" "*.Mask") (remove_unused_layers no) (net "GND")
   (thermal_bridge_angle 90))
  (pad "9" thru_hole circle (at 17.226 -1.283) (size 1.6 1.6) (drill 1) (layers "*.Cu" "*.Mask") (remove_unused_layers no) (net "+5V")
   (thermal_bridge_angle 90)))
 (segment (start 199.26 143.99066) (end 198.65416 144.5965) (width 0.2) (layer "F.Cu") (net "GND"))
 (segment (start 175.0604 144.5965) (end 173.8104 143.3465) (width 0.2) (layer "F.Cu") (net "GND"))
 (segment (start 199.26 142.93) (end 199.26 143.99066) (width 0.2) (layer "F.Cu") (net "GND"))
 (segment (start 198.65416 144.5965) (end 175.0604 144.5965) (width 0.2) (layer "F.Cu") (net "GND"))
 (segment (start 191.2104 122.0096) (end 191.2104 122.2885) (width 0.2) (layer "F.Cu") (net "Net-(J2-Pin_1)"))
 (segment (start 191.69 121.53) (end 191.2104 122.0096) (width 0.2) (layer "F.Cu") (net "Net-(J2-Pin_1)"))
 (segment (start 194.26 121.53) (end 191.69 121.53) (width 0.2) (layer "F.Cu") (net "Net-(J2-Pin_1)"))
 (segment (start 204.26 121.53) (end 205.585 120.205) (width 0.2) (layer "F.Cu") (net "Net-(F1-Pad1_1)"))
 (segment (start 205.585 120.205) (end 205.585 120.087793) (width 0.2) (layer "F.Cu") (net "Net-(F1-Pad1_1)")))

